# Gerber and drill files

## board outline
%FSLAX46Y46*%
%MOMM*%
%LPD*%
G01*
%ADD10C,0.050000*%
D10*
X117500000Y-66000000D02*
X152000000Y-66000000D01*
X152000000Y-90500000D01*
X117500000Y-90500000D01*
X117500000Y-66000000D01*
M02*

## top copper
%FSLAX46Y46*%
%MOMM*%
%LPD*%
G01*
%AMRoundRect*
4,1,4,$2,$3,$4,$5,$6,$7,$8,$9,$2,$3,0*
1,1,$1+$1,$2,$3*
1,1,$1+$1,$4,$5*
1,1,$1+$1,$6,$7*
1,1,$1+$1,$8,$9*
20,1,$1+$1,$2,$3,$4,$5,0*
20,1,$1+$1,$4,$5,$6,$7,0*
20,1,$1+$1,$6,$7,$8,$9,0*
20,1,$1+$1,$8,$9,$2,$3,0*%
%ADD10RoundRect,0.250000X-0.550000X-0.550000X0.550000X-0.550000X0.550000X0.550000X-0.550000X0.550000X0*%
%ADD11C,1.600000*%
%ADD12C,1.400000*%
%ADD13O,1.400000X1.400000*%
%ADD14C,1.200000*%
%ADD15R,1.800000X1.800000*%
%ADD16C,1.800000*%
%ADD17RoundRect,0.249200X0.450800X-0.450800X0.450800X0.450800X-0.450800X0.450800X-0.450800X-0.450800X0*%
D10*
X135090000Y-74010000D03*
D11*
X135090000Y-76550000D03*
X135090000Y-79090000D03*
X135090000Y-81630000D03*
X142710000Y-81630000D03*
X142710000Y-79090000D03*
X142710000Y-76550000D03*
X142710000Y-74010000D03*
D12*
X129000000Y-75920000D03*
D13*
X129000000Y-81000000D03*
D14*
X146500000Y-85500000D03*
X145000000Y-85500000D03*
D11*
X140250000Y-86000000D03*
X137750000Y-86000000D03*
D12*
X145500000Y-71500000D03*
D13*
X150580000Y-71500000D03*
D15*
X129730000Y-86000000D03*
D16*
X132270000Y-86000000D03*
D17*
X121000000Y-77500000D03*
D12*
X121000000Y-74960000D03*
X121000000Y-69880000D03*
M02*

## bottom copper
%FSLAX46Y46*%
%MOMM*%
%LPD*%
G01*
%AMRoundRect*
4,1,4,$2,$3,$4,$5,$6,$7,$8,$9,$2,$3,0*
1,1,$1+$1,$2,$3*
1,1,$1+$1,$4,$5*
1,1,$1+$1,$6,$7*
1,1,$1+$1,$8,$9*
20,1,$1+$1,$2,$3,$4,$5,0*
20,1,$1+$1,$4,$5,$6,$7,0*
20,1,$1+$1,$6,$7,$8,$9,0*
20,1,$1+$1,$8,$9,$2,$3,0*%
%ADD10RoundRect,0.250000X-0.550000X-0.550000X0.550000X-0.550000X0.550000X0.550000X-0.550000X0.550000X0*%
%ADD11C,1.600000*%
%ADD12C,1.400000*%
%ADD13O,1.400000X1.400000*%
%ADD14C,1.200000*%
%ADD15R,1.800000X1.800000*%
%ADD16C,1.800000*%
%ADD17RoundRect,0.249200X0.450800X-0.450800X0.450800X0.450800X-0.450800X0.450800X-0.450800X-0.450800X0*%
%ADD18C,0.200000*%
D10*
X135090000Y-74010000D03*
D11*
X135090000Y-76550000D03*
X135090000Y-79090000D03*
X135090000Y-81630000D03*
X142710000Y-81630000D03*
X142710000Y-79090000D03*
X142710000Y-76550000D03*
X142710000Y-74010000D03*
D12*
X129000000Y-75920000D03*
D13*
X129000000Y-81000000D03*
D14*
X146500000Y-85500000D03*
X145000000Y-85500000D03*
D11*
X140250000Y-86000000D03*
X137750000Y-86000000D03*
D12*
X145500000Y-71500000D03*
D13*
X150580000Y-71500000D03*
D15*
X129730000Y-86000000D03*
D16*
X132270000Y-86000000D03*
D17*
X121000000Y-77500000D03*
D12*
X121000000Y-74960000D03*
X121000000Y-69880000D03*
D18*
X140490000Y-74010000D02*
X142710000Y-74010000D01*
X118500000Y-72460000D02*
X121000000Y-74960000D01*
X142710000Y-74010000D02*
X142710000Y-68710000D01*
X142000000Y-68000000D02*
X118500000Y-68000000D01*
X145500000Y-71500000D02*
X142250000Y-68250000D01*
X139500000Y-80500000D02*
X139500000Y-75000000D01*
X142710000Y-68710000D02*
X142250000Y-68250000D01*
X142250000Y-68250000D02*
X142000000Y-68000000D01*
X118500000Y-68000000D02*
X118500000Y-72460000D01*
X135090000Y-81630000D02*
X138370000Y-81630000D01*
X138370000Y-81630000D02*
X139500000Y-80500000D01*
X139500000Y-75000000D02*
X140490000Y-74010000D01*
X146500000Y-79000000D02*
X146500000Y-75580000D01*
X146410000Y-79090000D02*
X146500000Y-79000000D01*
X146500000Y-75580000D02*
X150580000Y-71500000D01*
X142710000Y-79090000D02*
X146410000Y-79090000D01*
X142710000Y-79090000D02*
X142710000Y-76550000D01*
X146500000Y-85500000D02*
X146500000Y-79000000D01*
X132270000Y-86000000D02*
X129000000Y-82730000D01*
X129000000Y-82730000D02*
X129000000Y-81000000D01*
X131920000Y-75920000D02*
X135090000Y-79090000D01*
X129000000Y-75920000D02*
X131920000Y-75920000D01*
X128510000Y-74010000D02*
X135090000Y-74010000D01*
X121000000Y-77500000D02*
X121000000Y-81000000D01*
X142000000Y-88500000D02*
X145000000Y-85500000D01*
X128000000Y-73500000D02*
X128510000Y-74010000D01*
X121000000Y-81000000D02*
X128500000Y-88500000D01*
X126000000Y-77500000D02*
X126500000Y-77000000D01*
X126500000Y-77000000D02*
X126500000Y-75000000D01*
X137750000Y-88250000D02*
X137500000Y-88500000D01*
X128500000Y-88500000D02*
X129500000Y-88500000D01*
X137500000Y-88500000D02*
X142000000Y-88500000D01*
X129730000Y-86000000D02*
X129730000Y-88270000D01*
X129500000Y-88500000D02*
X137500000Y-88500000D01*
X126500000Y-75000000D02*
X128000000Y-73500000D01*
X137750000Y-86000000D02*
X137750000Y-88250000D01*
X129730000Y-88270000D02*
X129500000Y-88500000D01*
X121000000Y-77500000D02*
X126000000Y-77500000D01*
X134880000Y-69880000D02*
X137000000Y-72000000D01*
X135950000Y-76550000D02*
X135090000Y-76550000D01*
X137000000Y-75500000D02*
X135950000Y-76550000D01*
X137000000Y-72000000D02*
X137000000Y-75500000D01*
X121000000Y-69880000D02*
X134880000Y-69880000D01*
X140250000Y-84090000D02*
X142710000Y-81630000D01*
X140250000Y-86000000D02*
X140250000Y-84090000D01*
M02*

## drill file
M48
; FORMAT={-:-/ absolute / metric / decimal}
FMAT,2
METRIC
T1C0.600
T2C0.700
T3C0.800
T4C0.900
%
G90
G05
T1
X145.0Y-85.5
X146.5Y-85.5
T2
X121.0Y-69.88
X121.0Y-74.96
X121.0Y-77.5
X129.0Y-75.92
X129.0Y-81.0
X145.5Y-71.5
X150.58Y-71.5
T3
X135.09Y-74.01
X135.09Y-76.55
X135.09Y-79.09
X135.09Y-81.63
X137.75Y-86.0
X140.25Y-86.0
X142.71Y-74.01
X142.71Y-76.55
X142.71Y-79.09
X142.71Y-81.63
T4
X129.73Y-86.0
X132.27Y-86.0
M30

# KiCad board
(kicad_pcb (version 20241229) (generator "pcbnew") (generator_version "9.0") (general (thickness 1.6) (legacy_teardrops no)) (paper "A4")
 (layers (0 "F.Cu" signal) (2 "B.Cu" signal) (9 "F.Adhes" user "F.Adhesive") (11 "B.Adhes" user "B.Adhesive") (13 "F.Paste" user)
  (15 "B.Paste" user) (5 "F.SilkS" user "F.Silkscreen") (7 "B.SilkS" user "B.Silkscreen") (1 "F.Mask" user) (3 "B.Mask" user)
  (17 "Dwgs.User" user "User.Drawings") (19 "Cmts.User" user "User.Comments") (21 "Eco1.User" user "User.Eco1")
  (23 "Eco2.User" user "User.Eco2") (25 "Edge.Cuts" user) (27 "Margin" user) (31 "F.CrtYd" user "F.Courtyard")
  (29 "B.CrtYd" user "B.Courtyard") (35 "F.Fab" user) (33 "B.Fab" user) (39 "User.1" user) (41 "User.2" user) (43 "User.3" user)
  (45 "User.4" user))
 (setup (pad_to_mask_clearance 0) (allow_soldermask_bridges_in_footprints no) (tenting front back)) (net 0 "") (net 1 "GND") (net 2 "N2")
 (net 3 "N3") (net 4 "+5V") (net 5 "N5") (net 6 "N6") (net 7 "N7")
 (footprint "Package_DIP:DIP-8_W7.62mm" (layer "F.Cu") (at 135.09 74.01)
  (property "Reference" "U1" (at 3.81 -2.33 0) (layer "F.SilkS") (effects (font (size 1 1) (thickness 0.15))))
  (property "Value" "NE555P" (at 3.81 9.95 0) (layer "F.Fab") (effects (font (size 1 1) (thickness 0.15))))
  (pad "1" thru_hole roundrect (at 0 0) (size 1.6 1.6) (drill 0.8) (layers "*.Cu" "*.Mask") (remove_unused_layers no)
   (roundrect_rratio 0.15625) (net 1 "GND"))
  (pad "2" thru_hole circle (at 0 2.54) (size 1.6 1.6) (drill 0.8) (layers "*.Cu" "*.Mask") (remove_unused_layers no) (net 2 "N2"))
  (pad "3" thru_hole circle (at 0 5.08) (size 1.6 1.6) (drill 0.8) (layers "*.Cu" "*.Mask") (remove_unused_layers no) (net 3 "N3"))
  (pad "4" thru_hole circle (at 0 7.62) (size 1.6 1.6) (drill 0.8) (layers "*.Cu" "*.Mask") (remove_unused_layers no) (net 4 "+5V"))
  (pad "5" thru_hole circle (at 7.62 7.62) (size 1.6 1.6) (drill 0.8) (layers "*.Cu" "*.Mask") (remove_unused_layers no) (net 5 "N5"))
  (pad "6" thru_hole circle (at 7.62 5.08) (size 1.6 1.6) (drill 0.8) (layers "*.Cu" "*.Mask") (remove_unused_layers no) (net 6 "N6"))
  (pad "7" thru_hole circle (at 7.62 2.54) (size 1.6 1.6) (drill 0.8) (layers "*.Cu" "*.Mask") (remove_unused_layers no) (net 6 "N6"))
  (pad "8" thru_hole circle (at 7.62 0) (size 1.6 1.6) (drill 0.8) (layers "*.Cu" "*.Mask") (remove_unused_layers no) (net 4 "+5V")))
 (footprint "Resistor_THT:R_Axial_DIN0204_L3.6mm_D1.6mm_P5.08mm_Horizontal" (layer "F.Cu") (at 129 75.92 -90)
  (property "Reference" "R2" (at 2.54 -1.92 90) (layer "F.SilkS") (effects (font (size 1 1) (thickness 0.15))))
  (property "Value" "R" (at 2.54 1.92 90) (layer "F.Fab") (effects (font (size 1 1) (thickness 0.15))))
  (pad "1" thru_hole circle (at 0 0 270) (size 1.4 1.4) (drill 0.7) (layers "*.Cu" "*.Mask") (remove_unused_layers no) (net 3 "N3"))
  (pad "2" thru_hole oval (at 5.08 0 270) (size 1.4 1.4) (drill 0.7) (layers "*.Cu" "*.Mask") (remove_unused_layers no) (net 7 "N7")))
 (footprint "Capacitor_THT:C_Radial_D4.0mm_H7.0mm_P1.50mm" (layer "F.Cu") (at 146.5 85.5 180)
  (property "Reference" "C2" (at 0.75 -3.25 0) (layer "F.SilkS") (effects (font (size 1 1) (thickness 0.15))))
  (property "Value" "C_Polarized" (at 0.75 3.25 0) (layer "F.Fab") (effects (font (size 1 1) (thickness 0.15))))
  (pad "1" thru_hole circle (at 0 0 180) (size 1.2 1.2) (drill 0.6) (layers "*.Cu" "*.Mask") (remove_unused_layers no) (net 6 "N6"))
  (pad "2" thru_hole circle (at 1.5 0 180) (size 1.2 1.2) (drill 0.6) (layers "*.Cu" "*.Mask") (remove_unused_layers no) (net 1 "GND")))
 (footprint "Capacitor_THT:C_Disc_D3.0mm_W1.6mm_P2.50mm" (layer "F.Cu") (at 140.25 86 180)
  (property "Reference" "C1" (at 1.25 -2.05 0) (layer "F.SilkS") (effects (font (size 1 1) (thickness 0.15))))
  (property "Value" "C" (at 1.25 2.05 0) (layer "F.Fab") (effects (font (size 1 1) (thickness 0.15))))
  (pad "1" thru_hole circle (at 0 0 180) (size 1.6 1.6) (drill 0.8) (layers "*.Cu" "*.Mask") (remove_unused_layers no) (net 5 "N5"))
  (pad "2" thru_hole circle (at 2.5 0 180) (size 1.6 1.6) (drill 0.8) (layers "*.Cu" "*.Mask") (remove_unused_layers no) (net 1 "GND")))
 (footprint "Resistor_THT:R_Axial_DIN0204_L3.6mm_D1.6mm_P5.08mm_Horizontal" (layer "F.Cu") (at 145.5 71.5)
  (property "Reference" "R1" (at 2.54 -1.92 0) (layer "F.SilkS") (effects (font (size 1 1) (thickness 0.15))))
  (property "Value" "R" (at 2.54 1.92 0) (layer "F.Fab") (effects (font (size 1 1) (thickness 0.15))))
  (pad "1" thru_hole circle (at 0 0) (size 1.4 1.4) (drill 0.7) (layers "*.Cu" "*.Mask") (remove_unused_layers no) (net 4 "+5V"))
  (pad "2" thru_hole oval (at 5.08 0) (size 1.4 1.4) (drill 0.7) (layers "*.Cu" "*.Mask") (remove_unused_layers no) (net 6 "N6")))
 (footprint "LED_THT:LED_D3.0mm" (layer "F.Cu") (at 129.73 86)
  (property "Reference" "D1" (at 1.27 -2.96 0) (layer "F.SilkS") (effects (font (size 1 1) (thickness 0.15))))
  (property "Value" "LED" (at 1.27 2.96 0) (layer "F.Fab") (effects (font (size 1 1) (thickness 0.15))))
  (pad "1" thru_hole rect (at 0 0) (size 1.8 1.8) (drill 0.9) (layers "*.Cu" "*.Mask") (remove_unused_layers no) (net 1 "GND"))
  (pad "2" thru_hole circle (at 2.54 0) (size 1.8 1.8) (drill 0.9) (layers "*.Cu" "*.Mask") (remove_unused_layers no) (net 7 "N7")))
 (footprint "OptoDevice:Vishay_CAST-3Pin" (layer "F.Cu") (at 121 77.5 90)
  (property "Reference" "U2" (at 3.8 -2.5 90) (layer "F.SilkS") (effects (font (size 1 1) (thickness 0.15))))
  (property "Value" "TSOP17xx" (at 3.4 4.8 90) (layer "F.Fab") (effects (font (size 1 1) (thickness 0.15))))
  (pad "1" thru_hole roundrect (at 0 0 90) (size 1.4 1.4) (drill 0.7) (layers "*.Cu" "*.Mask") (remove_unused_layers no)
   (roundrect_rratio 0.178) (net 1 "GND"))
  (pad "2" thru_hole circle (at 2.54 0 90) (size 1.4 1.4) (drill 0.7) (layers "*.Cu" "*.Mask") (remove_unused_layers no) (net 4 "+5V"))
  (pad "3" thru_hole circle (at 7.62 0 90) (size 1.4 1.4) (drill 0.7) (layers "*.Cu" "*.Mask") (remove_unused_layers no) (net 2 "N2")))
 (gr_rect (start 117.5 66) (end 152 90.5) (stroke (width 0.05) (type default)) (fill no) (layer "Edge.Cuts"))
 (segment (start 140.49 74.01) (end 142.71 74.01) (width 0.2) (layer "B.Cu") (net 4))
 (segment (start 118.5 72.46) (end 121 74.96) (width 0.2) (layer "B.Cu") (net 4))
 (segment (start 142.71 74.01) (end 142.71 68.71) (width 0.2) (layer "B.Cu") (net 4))
 (segment (start 142 68) (end 118.5 68) (width 0.2) (layer "B.Cu") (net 4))
 (segment (start 145.5 71.5) (end 142.25 68.25) (width 0.2) (layer "B.Cu") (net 4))
 (segment (start 139.5 80.5) (end 139.5 75) (width 0.2) (layer "B.Cu") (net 4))
 (segment (start 142.71 68.71) (end 142.25 68.25) (width 0.2) (layer "B.Cu") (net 4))
 (segment (start 142.25 68.25) (end 142 68) (width 0.2) (layer "B.Cu") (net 4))
 (segment (start 118.5 68) (end 118.5 72.46) (width 0.2) (layer "B.Cu") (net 4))
 (segment (start 135.09 81.63) (end 138.37 81.63) (width 0.2) (layer "B.Cu") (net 4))
 (segment (start 138.37 81.63) (end 139.5 80.5) (width 0.2) (layer "B.Cu") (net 4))
 (segment (start 139.5 75) (end 140.49 74.01) (width 0.2) (layer "B.Cu") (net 4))
 (segment (start 146.5 79) (end 146.5 75.58) (width 0.2) (layer "B.Cu") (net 6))
 (segment (start 146.41 79.09) (end 146.5 79) (width 0.2) (layer "B.Cu") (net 6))
 (segment (start 146.5 75.58) (end 150.58 71.5) (width 0.2) (layer "B.Cu") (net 6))
 (segment (start 142.71 79.09) (end 146.41 79.09) (width 0.2) (layer "B.Cu") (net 6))
 (segment (start 142.71 79.09) (end 142.71 76.55) (width 0.2) (layer "B.Cu") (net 6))
 (segment (start 146.5 85.5) (end 146.5 79) (width 0.2) (layer "B.Cu") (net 6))
 (segment (start 132.27 86) (end 129 82.73) (width 0.2) (layer "B.Cu") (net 7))
 (segment (start 129 82.73) (end 129 81) (width 0.2) (layer "B.Cu") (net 7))
 (segment (start 131.92 75.92) (end 135.09 79.09) (width 0.2) (layer "B.Cu") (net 3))
 (segment (start 129 75.92) (end 131.92 75.92) (width 0.2) (layer "B.Cu") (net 3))
 (segment (start 128.51 74.01) (end 135.09 74.01) (width 0.2) (layer "B.Cu") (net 1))
 (segment (start 121 77.5) (end 121 81) (width 0.2) (layer "B.Cu") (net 1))
 (segment (start 142 88.5) (end 145 85.5) (width 0.2) (layer "B.Cu") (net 1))
 (segment (start 128 73.5) (end 128.51 74.01) (width 0.2) (layer "B.Cu") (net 1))
 (segment (start 121 81) (end 128.5 88.5) (width 0.2) (layer "B.Cu") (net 1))
 (segment (start 126 77.5) (end 126.5 77) (width 0.2) (layer "B.Cu") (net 1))
 (segment (start 126.5 77) (end 126.5 75) (width 0.2) (layer "B.Cu") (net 1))
 (segment (start 137.75 88.25) (end 137.5 88.5) (width 0.2) (layer "B.Cu") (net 1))
 (segment (start 128.5 88.5) (end 129.5 88.5) (width 0.2) (layer "B.Cu") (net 1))
 (segment (start 137.5 88.5) (end 142 88.5) (width 0.2) (layer "B.Cu") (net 1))
 (segment (start 129.73 86) (end 129.73 88.27) (width 0.2) (layer "B.Cu") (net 1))
 (segment (start 129.5 88.5) (end 137.5 88.5) (width 0.2) (layer "B.Cu") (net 1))
 (segment (start 126.5 75) (end 128 73.5) (width 0.2) (layer "B.Cu") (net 1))
 (segment (start 137.75 86) (end 137.75 88.25) (width 0.2) (layer "B.Cu") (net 1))
 (segment (start 129.73 88.27) (end 129.5 88.5) (width 0.2) (layer "B.Cu") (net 1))
 (segment (start 121 77.5) (end 126 77.5) (width 0.2) (layer "B.Cu") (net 1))
 (segment (start 134.88 69.88) (end 137 72) (width 0.2) (layer "B.Cu") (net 2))
 (segment (start 135.95 76.55) (end 135.09 76.55) (width 0.2) (layer "B.Cu") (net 2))
 (segment (start 137 75.5) (end 135.95 76.55) (width 0.2) (layer "B.Cu") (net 2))
 (segment (start 137 72) (end 137 75.5) (width 0.2) (layer "B.Cu") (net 2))
 (segment (start 121 69.88) (end 134.88 69.88) (width 0.2) (layer "B.Cu") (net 2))
 (segment (start 140.25 84.09) (end 142.71 81.63) (width 0.2) (layer "B.Cu") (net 5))
 (segment (start 140.25 86) (end 140.25 84.09) (width 0.2) (layer "B.Cu") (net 5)))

